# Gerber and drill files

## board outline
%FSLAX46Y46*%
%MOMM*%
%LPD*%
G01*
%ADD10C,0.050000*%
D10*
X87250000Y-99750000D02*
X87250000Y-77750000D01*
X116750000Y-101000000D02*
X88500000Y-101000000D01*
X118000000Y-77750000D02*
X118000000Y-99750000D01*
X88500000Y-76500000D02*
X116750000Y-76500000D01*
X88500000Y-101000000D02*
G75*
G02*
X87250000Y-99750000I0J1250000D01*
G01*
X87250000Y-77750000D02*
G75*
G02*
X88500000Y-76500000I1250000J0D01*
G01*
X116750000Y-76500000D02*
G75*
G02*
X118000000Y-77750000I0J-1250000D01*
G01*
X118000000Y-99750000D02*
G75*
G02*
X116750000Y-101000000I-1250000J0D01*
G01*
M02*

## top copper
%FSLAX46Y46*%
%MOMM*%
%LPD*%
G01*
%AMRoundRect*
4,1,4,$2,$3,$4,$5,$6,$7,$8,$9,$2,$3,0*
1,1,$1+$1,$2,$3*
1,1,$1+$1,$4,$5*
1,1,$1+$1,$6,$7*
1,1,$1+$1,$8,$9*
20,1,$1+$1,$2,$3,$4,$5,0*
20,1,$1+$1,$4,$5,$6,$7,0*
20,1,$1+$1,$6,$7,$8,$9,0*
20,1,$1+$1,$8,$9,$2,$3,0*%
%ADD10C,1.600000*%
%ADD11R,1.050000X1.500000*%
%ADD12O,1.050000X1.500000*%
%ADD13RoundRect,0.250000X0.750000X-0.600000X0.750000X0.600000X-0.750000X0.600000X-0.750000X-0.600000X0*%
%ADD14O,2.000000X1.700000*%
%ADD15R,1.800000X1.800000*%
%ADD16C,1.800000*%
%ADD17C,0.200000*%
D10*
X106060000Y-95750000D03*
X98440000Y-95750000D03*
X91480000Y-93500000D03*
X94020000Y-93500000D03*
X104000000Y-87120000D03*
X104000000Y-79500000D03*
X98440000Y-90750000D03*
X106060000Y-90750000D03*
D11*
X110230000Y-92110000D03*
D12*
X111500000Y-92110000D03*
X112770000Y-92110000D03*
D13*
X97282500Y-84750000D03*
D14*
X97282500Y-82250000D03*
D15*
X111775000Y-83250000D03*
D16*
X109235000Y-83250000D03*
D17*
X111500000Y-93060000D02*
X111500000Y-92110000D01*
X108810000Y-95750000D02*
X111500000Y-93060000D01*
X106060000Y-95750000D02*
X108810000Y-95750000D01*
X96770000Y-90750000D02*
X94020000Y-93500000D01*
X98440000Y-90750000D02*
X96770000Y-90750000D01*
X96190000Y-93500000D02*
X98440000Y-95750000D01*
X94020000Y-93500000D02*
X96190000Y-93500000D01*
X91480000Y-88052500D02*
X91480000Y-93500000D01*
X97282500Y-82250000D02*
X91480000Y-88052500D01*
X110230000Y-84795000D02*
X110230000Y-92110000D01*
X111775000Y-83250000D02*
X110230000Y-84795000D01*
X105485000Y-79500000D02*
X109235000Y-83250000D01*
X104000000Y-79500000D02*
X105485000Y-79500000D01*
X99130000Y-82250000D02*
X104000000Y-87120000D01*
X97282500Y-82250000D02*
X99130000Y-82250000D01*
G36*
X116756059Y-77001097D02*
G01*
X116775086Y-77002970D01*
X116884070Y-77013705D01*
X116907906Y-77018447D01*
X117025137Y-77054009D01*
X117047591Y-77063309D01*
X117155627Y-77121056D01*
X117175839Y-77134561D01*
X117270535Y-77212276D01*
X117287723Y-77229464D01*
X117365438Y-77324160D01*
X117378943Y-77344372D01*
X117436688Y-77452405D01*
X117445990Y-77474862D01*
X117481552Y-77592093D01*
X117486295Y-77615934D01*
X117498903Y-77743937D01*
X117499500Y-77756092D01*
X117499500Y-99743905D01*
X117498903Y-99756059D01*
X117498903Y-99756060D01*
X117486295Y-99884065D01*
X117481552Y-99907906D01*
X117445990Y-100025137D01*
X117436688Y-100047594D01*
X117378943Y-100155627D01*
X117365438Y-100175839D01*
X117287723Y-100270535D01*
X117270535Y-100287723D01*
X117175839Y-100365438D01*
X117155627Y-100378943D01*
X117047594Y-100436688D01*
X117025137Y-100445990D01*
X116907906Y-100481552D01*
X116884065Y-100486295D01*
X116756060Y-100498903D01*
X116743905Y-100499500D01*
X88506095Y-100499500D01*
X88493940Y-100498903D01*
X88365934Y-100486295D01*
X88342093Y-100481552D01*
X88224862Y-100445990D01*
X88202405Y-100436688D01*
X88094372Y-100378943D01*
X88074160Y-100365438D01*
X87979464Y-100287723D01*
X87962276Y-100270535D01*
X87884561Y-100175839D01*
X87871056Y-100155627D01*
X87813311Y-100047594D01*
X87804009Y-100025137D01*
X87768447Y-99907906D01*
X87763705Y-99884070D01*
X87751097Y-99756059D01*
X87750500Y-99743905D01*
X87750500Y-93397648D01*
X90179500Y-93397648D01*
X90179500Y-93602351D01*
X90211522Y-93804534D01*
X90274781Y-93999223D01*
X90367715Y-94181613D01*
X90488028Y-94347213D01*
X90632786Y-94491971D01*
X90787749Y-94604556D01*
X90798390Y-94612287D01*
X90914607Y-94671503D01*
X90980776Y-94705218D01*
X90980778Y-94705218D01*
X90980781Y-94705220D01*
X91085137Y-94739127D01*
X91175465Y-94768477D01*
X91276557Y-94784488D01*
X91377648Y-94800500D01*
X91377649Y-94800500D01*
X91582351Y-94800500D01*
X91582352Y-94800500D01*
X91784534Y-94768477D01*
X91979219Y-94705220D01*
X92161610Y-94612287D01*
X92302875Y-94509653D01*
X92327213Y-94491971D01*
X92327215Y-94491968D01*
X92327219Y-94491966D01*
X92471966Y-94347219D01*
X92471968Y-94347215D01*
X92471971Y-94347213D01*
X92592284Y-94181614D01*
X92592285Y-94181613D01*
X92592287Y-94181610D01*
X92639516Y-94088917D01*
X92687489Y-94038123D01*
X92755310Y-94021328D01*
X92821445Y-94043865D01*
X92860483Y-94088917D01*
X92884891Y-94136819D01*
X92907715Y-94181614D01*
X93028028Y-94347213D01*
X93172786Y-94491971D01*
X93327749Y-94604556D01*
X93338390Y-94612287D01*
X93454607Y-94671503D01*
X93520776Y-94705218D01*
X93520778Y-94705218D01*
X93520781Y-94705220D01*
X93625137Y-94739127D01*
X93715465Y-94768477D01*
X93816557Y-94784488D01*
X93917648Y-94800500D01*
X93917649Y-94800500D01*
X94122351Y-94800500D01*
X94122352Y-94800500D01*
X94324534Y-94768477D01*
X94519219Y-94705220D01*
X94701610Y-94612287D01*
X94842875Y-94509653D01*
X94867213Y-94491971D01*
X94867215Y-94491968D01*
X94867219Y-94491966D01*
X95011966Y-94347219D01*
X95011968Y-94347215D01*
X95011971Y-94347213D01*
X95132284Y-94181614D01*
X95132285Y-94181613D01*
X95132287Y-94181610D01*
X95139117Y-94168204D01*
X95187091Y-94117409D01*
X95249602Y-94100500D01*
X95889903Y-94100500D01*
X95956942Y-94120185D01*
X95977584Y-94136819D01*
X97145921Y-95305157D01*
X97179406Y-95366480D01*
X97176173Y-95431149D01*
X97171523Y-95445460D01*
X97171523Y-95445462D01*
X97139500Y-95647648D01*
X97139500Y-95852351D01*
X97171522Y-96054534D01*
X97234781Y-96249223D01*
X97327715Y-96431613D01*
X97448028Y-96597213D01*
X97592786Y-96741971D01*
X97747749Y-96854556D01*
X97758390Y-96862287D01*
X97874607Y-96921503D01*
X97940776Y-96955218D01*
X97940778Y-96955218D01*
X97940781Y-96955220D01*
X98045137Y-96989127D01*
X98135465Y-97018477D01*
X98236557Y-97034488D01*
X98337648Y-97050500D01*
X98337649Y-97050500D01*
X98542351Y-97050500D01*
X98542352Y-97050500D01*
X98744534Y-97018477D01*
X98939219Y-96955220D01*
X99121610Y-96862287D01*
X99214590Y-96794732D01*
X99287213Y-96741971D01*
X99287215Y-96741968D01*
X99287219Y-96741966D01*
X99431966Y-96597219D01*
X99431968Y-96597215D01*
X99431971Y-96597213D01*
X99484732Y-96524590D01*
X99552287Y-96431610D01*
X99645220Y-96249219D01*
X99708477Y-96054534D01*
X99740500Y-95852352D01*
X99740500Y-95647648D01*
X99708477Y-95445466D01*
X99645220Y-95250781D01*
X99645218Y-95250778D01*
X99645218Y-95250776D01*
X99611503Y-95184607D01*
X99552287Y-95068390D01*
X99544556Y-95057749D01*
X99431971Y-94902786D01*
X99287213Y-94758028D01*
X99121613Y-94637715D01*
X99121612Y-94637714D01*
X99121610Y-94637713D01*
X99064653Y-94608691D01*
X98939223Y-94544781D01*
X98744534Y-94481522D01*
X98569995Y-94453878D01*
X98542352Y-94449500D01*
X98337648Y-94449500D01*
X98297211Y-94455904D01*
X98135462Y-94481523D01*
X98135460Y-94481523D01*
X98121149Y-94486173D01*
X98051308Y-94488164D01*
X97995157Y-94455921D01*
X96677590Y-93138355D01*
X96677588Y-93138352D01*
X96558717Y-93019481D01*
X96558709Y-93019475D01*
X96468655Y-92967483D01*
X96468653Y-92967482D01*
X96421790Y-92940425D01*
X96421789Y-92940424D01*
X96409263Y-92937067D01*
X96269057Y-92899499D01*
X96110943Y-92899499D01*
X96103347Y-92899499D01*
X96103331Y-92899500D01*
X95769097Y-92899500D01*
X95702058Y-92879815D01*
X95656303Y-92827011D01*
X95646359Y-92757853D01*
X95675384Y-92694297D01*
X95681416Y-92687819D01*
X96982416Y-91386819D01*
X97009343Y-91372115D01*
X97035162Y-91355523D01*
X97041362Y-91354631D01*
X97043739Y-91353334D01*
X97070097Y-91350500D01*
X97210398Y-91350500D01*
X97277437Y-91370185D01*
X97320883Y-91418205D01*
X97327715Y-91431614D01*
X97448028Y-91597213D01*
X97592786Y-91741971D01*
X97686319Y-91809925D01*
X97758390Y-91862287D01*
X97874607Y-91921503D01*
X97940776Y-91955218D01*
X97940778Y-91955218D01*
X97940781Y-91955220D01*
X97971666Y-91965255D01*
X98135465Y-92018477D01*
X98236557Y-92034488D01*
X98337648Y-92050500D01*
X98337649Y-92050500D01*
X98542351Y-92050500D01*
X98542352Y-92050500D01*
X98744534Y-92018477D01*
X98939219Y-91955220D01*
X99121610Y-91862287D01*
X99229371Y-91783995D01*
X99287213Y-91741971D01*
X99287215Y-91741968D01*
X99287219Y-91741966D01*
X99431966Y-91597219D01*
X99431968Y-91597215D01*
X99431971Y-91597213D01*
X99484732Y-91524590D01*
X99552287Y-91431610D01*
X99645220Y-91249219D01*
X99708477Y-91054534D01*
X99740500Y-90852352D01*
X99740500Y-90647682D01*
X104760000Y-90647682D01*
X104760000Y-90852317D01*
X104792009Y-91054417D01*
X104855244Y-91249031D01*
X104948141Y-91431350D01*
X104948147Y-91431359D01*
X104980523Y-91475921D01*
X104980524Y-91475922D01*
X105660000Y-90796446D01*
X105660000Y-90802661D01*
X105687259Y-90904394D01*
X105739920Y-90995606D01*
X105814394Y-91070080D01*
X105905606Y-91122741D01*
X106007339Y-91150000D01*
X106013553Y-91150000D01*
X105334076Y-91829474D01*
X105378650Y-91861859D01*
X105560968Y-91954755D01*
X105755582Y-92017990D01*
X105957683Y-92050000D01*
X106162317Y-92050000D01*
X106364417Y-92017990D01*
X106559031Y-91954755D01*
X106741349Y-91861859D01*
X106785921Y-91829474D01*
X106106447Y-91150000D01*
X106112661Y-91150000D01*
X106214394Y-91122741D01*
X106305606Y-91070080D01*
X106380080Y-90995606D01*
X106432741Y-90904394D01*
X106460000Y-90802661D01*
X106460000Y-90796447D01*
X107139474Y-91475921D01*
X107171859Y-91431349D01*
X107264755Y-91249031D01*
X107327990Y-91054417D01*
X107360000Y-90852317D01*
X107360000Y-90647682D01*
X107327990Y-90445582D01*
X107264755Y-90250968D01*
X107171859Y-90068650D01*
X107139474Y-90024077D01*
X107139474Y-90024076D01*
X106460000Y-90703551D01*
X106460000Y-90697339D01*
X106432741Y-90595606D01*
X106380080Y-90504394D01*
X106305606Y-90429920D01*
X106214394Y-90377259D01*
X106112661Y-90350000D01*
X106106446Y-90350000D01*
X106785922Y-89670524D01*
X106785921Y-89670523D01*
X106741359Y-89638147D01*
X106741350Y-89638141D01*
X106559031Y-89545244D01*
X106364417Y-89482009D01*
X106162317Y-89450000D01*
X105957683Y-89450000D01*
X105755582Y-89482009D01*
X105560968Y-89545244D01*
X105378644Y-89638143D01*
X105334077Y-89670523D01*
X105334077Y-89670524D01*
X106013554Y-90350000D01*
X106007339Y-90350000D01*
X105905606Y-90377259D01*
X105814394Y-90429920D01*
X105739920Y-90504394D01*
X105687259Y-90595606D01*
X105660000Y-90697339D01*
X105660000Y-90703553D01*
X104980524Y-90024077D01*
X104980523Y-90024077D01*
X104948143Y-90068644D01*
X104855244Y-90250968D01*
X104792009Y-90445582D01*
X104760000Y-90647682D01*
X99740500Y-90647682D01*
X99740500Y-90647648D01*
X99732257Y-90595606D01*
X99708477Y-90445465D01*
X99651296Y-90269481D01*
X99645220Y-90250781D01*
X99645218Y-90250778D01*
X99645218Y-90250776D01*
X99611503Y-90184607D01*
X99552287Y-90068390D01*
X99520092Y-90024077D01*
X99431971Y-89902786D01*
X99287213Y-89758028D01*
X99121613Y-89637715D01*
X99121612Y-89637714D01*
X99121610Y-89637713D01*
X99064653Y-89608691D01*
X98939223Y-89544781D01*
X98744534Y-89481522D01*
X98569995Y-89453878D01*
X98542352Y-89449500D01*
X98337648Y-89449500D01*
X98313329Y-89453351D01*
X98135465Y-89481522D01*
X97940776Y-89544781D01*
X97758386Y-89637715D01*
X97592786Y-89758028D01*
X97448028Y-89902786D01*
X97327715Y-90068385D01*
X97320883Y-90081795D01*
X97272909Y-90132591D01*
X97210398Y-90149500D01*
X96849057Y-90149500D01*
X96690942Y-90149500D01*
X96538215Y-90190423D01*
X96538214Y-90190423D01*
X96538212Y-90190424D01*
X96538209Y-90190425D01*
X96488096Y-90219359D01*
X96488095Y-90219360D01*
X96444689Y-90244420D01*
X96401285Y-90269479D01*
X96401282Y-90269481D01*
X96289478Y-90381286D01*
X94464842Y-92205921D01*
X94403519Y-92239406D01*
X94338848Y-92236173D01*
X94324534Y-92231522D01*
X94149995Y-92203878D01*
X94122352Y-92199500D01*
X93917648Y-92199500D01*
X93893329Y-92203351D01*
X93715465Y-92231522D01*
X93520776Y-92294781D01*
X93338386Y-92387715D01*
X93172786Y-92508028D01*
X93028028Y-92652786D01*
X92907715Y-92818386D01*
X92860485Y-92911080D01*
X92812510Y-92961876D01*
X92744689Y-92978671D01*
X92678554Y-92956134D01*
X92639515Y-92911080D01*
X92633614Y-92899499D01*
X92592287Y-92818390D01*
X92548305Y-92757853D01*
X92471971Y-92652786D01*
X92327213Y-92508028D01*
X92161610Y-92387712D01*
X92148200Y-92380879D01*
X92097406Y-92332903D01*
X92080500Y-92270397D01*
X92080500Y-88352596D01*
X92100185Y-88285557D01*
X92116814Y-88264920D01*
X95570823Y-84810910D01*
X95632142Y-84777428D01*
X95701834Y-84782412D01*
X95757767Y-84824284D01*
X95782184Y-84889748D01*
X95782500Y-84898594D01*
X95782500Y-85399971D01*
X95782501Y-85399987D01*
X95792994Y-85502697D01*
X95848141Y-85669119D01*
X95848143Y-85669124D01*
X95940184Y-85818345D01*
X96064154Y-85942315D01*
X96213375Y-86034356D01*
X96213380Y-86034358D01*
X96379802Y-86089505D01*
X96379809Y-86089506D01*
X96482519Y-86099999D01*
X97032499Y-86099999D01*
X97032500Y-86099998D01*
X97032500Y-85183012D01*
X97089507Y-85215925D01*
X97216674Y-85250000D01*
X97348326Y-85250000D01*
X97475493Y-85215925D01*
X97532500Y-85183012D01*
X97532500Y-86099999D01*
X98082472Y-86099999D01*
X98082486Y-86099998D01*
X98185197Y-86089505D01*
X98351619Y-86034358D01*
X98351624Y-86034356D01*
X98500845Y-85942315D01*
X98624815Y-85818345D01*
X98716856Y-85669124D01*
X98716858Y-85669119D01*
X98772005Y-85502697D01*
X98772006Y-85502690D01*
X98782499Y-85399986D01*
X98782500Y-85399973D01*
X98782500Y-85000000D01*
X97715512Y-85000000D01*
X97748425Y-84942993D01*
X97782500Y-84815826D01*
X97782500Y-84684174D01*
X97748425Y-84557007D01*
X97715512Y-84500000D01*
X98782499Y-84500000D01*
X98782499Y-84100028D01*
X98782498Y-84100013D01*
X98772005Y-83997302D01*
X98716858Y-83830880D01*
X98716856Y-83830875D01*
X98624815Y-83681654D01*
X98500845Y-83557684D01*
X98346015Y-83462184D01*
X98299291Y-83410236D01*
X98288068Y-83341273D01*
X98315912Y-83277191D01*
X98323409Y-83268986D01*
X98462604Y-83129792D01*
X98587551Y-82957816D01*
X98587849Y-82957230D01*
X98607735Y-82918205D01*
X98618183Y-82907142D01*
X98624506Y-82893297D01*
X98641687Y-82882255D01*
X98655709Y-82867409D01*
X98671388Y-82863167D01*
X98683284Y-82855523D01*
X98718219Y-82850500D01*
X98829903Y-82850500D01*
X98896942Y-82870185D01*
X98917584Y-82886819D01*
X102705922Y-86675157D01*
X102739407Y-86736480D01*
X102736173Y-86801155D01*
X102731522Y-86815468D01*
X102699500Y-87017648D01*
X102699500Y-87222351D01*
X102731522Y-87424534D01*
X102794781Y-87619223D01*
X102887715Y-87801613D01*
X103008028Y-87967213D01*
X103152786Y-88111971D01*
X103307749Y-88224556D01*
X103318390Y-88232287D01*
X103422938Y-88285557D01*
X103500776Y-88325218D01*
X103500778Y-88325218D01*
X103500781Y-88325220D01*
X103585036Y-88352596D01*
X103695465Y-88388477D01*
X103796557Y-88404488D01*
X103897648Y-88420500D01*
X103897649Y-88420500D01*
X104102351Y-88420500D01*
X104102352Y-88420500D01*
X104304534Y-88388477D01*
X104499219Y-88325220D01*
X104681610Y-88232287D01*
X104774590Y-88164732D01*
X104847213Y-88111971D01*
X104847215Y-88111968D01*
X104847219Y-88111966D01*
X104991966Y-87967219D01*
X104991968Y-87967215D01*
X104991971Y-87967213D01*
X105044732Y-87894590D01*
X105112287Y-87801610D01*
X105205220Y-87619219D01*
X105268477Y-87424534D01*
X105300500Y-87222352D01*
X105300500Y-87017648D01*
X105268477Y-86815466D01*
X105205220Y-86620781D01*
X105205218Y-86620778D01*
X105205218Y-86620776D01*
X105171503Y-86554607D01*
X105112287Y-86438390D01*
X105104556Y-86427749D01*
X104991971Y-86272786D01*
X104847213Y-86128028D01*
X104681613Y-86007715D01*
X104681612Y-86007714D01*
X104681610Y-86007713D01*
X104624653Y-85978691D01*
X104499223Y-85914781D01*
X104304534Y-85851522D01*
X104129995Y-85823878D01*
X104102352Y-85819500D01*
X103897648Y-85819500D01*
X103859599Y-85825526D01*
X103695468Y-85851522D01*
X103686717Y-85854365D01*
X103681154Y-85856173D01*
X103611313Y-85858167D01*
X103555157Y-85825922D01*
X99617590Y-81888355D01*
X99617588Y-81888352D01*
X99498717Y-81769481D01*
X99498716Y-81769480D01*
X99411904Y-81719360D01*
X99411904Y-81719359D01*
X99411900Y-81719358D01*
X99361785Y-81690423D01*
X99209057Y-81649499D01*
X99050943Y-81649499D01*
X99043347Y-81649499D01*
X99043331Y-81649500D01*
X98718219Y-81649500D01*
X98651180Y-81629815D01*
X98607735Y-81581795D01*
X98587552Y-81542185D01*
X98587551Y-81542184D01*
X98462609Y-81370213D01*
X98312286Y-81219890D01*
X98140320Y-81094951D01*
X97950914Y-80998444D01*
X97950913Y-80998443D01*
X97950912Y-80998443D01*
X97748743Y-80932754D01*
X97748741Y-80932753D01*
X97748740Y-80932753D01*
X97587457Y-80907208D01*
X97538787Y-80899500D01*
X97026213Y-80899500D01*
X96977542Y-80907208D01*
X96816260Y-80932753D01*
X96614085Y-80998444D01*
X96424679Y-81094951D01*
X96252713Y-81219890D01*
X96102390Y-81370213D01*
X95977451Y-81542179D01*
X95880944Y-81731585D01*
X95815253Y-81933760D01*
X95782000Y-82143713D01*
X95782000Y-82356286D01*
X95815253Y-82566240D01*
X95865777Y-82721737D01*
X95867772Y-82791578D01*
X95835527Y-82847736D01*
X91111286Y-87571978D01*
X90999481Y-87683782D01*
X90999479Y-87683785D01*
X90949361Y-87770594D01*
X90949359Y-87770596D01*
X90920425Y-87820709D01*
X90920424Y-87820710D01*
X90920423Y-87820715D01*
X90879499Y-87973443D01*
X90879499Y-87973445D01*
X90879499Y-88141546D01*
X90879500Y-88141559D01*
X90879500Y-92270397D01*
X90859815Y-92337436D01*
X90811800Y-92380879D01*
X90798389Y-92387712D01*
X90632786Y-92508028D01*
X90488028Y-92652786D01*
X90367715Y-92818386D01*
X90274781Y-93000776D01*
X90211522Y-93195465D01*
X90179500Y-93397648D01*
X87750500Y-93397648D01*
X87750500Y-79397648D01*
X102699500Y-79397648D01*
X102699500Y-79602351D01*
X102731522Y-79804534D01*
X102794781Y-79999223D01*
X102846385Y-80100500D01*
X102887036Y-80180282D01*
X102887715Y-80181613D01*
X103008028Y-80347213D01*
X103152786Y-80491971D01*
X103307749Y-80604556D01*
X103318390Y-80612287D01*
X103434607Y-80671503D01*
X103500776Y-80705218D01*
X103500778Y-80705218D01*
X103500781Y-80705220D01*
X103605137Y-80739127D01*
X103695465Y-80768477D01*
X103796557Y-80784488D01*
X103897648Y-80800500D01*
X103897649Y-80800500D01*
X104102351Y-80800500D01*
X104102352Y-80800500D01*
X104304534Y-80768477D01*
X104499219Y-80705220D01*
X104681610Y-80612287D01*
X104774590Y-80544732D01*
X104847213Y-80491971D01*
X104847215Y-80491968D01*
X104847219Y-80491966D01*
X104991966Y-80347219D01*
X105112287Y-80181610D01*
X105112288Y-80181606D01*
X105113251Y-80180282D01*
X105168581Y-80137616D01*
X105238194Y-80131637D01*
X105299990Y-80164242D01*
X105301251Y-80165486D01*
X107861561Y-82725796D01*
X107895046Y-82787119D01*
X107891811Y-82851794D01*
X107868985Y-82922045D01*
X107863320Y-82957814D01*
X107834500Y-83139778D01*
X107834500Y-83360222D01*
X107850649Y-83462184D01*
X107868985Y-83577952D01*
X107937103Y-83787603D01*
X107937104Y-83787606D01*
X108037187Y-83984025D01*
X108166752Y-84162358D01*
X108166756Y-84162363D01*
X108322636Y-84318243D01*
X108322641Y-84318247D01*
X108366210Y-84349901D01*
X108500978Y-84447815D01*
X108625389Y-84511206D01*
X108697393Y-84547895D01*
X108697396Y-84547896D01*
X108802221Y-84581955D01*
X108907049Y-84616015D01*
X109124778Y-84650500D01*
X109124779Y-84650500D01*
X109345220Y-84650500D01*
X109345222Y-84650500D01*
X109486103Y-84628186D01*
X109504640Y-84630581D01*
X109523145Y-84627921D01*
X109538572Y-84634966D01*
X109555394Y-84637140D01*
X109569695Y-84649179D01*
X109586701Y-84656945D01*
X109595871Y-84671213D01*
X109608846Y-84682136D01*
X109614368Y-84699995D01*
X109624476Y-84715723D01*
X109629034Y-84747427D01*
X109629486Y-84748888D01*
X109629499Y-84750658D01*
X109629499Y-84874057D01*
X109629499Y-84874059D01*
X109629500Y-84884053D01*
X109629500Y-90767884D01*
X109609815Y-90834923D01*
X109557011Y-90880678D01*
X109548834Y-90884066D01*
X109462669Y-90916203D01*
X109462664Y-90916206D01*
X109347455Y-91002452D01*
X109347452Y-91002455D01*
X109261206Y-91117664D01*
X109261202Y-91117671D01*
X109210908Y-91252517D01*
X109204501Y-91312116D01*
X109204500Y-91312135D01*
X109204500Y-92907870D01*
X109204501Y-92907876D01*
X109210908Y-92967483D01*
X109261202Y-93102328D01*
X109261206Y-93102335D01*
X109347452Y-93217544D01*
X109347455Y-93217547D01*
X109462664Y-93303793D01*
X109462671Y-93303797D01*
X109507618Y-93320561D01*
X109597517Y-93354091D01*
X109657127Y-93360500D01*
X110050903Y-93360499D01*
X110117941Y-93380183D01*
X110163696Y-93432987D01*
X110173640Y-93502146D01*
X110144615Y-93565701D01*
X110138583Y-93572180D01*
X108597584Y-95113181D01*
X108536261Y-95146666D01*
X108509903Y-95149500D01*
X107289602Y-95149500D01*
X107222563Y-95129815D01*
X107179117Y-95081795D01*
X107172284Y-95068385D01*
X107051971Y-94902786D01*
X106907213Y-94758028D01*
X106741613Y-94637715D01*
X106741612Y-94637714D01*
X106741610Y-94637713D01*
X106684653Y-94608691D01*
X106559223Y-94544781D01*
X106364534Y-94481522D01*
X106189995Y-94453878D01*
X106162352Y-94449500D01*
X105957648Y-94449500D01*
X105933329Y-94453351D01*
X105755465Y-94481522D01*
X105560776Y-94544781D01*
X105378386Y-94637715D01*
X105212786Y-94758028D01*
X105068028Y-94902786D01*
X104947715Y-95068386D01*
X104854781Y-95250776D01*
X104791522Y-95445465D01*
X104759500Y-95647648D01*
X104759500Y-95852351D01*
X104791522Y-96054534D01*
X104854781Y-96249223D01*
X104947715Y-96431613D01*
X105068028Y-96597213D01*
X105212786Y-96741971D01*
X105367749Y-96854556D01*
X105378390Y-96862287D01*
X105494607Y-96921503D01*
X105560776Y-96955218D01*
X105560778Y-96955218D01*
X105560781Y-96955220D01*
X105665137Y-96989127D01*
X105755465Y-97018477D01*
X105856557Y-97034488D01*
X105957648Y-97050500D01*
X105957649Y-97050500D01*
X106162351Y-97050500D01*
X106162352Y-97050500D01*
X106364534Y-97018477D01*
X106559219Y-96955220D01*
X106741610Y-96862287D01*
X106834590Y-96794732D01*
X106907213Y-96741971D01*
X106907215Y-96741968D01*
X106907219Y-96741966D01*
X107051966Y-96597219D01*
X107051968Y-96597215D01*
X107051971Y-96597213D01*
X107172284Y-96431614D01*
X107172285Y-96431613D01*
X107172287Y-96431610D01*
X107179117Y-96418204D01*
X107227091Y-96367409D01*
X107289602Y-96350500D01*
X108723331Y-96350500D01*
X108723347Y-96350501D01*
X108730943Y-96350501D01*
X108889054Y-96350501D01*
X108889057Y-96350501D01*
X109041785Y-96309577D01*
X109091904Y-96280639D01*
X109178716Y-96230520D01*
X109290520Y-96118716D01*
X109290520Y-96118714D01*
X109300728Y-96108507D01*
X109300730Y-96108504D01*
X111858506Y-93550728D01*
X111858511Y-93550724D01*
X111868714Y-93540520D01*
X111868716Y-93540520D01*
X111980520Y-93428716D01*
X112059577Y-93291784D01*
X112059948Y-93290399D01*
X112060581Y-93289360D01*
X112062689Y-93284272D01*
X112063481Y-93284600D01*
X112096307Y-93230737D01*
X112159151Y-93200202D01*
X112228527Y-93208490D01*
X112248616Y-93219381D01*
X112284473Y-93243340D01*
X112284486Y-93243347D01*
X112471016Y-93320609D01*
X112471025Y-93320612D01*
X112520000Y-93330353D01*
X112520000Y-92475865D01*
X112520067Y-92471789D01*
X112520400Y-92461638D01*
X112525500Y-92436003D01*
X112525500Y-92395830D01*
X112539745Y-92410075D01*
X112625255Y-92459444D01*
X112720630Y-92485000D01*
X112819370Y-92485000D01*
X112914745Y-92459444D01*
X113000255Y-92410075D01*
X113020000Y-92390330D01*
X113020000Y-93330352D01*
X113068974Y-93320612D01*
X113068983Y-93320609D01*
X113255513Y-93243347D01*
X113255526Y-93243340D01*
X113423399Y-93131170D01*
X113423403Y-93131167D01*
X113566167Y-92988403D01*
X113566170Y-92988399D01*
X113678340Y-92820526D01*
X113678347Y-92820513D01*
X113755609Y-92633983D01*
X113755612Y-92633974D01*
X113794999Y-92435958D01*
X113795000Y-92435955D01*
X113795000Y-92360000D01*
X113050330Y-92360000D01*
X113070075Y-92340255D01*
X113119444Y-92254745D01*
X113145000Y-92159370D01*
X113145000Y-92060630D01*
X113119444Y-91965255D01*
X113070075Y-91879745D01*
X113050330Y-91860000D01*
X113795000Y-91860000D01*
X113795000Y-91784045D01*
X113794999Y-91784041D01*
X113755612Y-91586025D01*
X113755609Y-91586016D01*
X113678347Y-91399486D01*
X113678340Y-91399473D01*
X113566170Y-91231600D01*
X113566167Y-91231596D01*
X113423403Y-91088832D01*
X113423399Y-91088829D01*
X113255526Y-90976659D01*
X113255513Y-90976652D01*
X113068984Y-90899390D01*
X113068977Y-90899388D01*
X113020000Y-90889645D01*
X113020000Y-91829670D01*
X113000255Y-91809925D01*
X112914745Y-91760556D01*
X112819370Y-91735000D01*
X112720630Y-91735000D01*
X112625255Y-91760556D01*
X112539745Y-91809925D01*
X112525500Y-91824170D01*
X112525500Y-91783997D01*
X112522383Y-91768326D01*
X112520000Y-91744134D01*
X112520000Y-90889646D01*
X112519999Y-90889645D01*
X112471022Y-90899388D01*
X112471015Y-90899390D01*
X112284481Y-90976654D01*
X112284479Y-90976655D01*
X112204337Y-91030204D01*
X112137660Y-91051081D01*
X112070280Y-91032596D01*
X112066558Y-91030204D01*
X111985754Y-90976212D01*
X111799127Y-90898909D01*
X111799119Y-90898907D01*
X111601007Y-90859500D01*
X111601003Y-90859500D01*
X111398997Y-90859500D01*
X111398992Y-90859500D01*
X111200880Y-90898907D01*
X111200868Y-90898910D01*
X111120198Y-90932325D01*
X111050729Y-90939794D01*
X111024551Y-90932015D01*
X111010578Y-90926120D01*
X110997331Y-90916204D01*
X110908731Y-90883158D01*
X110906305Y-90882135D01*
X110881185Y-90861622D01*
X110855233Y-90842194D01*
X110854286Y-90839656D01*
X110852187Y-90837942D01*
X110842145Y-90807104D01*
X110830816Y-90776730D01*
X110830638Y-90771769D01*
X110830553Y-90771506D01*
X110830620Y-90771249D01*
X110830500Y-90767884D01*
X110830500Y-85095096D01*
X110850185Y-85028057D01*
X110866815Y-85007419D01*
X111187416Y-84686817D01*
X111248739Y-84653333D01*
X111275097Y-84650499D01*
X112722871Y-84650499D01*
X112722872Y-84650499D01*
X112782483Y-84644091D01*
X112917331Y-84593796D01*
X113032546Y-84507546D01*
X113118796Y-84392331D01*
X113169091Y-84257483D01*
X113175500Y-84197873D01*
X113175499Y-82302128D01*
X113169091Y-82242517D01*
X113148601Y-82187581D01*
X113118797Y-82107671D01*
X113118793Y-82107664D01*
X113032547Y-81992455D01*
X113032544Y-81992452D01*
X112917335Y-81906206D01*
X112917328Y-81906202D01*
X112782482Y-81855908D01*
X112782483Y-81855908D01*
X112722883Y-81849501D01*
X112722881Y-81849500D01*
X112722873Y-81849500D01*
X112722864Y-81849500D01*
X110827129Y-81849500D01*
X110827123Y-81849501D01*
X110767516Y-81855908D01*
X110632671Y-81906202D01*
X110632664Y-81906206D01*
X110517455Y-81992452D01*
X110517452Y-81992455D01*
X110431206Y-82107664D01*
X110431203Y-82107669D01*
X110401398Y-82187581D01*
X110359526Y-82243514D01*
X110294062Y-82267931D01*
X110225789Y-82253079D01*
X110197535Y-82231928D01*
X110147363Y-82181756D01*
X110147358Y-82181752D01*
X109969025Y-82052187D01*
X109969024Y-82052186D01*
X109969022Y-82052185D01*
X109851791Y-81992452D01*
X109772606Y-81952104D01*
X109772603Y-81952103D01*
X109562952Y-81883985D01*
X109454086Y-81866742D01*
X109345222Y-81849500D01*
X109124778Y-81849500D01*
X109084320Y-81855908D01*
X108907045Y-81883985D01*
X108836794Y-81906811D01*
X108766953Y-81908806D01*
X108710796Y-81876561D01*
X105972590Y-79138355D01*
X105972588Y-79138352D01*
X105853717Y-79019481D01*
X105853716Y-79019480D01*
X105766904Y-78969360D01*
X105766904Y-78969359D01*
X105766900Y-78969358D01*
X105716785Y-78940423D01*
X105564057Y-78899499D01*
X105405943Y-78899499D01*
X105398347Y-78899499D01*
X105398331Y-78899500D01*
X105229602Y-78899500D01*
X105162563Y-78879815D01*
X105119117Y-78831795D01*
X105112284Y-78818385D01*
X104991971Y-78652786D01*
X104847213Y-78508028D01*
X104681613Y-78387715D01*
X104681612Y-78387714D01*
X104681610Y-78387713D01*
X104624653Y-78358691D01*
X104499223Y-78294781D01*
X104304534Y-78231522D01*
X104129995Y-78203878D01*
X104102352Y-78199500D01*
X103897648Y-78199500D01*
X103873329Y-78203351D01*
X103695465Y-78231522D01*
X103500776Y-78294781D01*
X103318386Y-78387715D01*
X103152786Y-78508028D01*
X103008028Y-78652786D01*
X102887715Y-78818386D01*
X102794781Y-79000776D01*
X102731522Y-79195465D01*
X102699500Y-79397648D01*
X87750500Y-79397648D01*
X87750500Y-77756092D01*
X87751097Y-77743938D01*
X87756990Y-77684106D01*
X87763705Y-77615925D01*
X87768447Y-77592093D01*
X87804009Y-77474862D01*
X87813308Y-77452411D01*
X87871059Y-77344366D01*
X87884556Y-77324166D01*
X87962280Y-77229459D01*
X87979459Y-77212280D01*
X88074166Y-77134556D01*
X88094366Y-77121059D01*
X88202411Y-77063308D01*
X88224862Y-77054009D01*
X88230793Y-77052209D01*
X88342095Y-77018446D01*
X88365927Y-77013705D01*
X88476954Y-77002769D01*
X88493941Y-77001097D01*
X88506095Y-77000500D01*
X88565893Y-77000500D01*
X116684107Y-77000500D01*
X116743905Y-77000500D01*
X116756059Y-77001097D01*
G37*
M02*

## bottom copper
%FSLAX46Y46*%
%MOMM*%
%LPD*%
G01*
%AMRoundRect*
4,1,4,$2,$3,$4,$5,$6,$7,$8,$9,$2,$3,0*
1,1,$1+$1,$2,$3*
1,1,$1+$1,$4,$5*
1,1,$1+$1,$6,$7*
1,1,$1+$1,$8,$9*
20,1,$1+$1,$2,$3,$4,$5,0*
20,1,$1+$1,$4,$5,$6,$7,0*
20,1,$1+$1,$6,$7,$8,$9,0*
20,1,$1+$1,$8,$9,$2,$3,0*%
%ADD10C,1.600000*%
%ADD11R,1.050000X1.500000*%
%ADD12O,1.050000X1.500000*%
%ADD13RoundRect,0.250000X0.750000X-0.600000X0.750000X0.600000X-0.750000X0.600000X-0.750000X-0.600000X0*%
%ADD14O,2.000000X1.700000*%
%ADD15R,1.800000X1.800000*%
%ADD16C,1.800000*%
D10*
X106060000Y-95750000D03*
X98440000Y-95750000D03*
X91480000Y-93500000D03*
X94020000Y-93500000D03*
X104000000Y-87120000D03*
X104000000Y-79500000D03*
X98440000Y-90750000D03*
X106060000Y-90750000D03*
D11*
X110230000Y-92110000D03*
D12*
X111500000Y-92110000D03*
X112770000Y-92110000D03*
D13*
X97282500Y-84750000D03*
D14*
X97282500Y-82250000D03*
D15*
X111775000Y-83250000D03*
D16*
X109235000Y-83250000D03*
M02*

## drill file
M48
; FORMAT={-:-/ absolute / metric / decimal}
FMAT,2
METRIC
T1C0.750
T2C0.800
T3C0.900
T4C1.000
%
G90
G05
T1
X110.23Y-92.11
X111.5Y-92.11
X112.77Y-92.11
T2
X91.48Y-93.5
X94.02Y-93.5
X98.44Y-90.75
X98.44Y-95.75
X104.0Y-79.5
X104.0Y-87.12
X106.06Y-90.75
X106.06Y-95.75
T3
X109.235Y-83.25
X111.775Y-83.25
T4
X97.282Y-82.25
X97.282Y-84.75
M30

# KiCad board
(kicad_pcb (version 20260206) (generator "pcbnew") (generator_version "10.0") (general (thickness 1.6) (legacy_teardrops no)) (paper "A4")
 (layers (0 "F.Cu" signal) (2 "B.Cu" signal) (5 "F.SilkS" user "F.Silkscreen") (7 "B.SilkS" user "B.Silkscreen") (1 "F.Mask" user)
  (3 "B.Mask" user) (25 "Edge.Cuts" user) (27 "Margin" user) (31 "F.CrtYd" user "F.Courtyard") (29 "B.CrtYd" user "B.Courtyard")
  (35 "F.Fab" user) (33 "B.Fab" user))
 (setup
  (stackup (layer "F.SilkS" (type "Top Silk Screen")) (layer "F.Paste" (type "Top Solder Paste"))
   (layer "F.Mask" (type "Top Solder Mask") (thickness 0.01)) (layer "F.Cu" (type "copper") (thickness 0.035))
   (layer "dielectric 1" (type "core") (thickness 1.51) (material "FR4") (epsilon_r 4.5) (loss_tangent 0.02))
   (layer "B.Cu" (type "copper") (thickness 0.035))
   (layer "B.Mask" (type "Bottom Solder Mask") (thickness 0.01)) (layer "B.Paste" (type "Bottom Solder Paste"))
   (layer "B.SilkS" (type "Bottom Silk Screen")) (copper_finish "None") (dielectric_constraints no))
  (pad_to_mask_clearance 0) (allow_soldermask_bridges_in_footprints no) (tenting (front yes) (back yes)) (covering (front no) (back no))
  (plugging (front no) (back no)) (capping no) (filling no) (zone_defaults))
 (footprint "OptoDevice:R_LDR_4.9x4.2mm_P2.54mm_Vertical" (layer "F.Cu") (at 91.48 93.5)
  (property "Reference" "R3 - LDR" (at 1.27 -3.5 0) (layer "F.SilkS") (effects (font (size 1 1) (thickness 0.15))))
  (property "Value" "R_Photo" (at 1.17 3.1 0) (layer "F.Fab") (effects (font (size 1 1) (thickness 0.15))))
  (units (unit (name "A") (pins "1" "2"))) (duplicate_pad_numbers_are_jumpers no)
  (pad "1" thru_hole circle (at 0 0) (size 1.6 1.6) (drill 0.8) (layers "*.Cu" "*.Mask") (remove_unused_layers no) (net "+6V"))
  (pad "2" thru_hole circle (at 2.54 0) (size 1.6 1.6) (drill 0.8) (layers "*.Cu" "*.Mask") (remove_unused_layers no) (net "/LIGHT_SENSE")))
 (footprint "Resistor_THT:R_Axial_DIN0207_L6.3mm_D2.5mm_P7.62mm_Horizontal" (layer "F.Cu") (at 98.44 90.75)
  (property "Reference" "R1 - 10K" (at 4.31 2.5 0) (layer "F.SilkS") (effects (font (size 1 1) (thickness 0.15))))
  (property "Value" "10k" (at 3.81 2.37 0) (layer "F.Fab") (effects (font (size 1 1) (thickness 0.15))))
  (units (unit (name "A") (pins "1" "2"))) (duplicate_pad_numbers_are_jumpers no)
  (pad "1" thru_hole circle (at 0 0) (size 1.6 1.6) (drill 0.8) (layers "*.Cu" "*.Mask") (remove_unused_layers no) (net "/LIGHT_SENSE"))
  (pad "2" thru_hole circle (at 7.62 0) (size 1.6 1.6) (drill 0.8) (layers "*.Cu" "*.Mask") (remove_unused_layers no) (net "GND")))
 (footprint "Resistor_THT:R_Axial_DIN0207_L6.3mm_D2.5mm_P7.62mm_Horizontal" (layer "F.Cu") (at 104 87.12 90)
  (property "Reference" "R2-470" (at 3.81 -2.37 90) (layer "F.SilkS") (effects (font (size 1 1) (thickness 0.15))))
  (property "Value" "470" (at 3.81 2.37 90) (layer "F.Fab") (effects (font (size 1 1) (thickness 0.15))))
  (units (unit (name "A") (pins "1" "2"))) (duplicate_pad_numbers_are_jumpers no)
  (pad "1" thru_hole circle (at 0 0 90) (size 1.6 1.6) (drill 0.8) (layers "*.Cu" "*.Mask") (remove_unused_layers no) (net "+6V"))
  (pad "2" thru_hole circle (at 7.62 0 90) (size 1.6 1.6) (drill 0.8) (layers "*.Cu" "*.Mask") (remove_unused_layers no) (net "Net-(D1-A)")))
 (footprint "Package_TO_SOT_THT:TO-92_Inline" (layer "F.Cu") (at 110.23 92.11)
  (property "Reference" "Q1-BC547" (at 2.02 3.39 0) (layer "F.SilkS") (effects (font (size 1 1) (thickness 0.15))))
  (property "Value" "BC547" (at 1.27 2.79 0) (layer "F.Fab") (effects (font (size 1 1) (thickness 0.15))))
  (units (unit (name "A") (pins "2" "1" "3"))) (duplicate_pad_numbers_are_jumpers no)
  (pad "1" thru_hole rect (at 0 0) (size 1.05 1.5) (drill 0.75) (layers "*.Cu" "*.Mask") (remove_unused_layers no) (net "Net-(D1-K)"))
  (pad "2" thru_hole oval (at 1.27 0) (size 1.05 1.5) (drill 0.75) (layers "*.Cu" "*.Mask") (remove_unused_layers no) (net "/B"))
  (pad "3" thru_hole oval (at 2.54 0) (size 1.05 1.5) (drill 0.75) (layers "*.Cu" "*.Mask") (remove_unused_layers no) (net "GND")))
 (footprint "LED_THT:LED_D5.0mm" (layer "F.Cu") (at 111.775 83.25 180)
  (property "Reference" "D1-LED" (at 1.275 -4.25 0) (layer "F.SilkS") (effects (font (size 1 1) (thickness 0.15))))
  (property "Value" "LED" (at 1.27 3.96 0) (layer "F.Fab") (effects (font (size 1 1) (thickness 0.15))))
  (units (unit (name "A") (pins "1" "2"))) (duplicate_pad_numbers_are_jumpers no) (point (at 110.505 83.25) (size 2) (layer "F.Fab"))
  (pad "1" thru_hole rect (at 0 0 180) (size 1.8 1.8) (drill 0.9) (layers "*.Cu" "*.Mask") (remove_unused_layers no) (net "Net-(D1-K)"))
  (pad "2" thru_hole circle (at 2.54 0 180) (size 1.8 1.8) (drill 0.9) (layers "*.Cu" "*.Mask") (remove_unused_layers no) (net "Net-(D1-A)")))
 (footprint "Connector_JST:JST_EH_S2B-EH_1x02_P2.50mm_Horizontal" (layer "F.Cu") (at 97.2825 84.75 90)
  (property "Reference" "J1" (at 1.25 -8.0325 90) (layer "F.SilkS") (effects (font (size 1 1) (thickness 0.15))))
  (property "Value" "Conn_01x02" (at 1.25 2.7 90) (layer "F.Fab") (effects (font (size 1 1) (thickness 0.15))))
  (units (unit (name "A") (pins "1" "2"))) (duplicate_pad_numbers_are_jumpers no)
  (pad "1" thru_hole roundrect (at 0 0 90) (size 1.7 2) (drill 1) (layers "*.Cu" "*.Mask") (remove_unused_layers no)
   (roundrect_rratio 0.147059) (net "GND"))
  (pad "2" thru_hole oval (at 2.5 0 90) (size 1.7 2) (drill 1) (layers "*.Cu" "*.Mask") (remove_unused_layers no) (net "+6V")))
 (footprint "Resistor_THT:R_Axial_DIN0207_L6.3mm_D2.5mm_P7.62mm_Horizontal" (layer "F.Cu") (at 106.06 95.75 180)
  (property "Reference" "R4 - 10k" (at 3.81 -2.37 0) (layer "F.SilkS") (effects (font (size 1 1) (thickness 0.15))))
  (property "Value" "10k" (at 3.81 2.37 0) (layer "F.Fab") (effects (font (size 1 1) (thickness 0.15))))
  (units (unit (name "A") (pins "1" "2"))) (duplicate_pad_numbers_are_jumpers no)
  (pad "1" thru_hole circle (at 0 0 180) (size 1.6 1.6) (drill 0.8) (layers "*.Cu" "*.Mask") (remove_unused_layers no) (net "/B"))
  (pad "2" thru_hole circle (at 7.62 0 180) (size 1.6 1.6) (drill 0.8) (layers "*.Cu" "*.Mask") (remove_unused_layers no)
   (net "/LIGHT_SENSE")))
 (gr_arc (start 87.25 77.75) (mid 87.616117 76.866117) (end 88.5 76.5) (stroke (width 0.05) (type default)) (layer "Edge.Cuts"))
 (gr_line (start 87.25 99.75) (end 87.25 77.75) (stroke (width 0.05) (type default)) (layer "Edge.Cuts"))
 (gr_line (start 88.5 76.5) (end 116.75 76.5) (stroke (width 0.05) (type default)) (layer "Edge.Cuts"))
 (gr_arc (start 88.5 101) (mid 87.616117 100.633883) (end 87.25 99.75) (stroke (width 0.05) (type default)) (layer "Edge.Cuts"))
 (gr_arc (start 116.75 76.5) (mid 117.633883 76.866117) (end 118 77.75) (stroke (width 0.05) (type default)) (layer "Edge.Cuts"))
 (gr_line (start 116.75 101) (end 88.5 101) (stroke (width 0.05) (type default)) (layer "Edge.Cuts"))
 (gr_line (start 118 77.75) (end 118 99.75) (stroke (width 0.05) (type default)) (layer "Edge.Cuts"))
 (gr_arc (start 118 99.75) (mid 117.633883 100.633883) (end 116.75 101) (stroke (width 0.05) (type default)) (layer "Edge.Cuts"))
 (segment (start 105.485 79.5) (end 109.235 83.25) (width 0.2) (layer "F.Cu") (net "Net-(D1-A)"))
 (segment (start 104 79.5) (end 105.485 79.5) (width 0.2) (layer "F.Cu") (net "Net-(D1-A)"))
 (segment (start 111.775 83.25) (end 110.23 84.795) (width 0.2) (layer "F.Cu") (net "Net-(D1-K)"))
 (segment (start 110.23 84.795) (end 110.23 92.11) (width 0.2) (layer "F.Cu") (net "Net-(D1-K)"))
 (segment (start 91.48 88.0525) (end 91.48 93.5) (width 0.2) (layer "F.Cu") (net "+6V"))
 (segment (start 97.2825 82.25) (end 99.13 82.25) (width 0.2) (layer "F.Cu") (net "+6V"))
 (segment (start 97.2825 82.25) (end 91.48 88.0525) (width 0.2) (layer "F.Cu") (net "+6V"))
 (segment (start 99.13 82.25) (end 104 87.12) (width 0.2) (layer "F.Cu") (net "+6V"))
 (segment (start 111.5 93.06) (end 111.5 92.11) (width 0.2) (layer "F.Cu") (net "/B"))
 (segment (start 106.06 95.75) (end 108.81 95.75) (width 0.2) (layer "F.Cu") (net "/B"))
 (segment (start 108.81 95.75) (end 111.5 93.06) (width 0.2) (layer "F.Cu") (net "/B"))
 (segment (start 98.44 90.75) (end 96.77 90.75) (width 0.2) (layer "F.Cu") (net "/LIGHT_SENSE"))
 (segment (start 96.77 90.75) (end 94.02 93.5) (width 0.2) (layer "F.Cu") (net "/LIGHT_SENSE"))
 (segment (start 94.02 93.5) (end 96.19 93.5) (width 0.2) (layer "F.Cu") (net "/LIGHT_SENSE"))
 (segment (start 96.19 93.5) (end 98.44 95.75) (width 0.2) (layer "F.Cu") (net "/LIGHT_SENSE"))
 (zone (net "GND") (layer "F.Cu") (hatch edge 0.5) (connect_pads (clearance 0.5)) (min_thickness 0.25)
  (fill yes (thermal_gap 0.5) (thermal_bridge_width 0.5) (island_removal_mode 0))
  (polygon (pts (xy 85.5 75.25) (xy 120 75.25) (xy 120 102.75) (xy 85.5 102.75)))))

